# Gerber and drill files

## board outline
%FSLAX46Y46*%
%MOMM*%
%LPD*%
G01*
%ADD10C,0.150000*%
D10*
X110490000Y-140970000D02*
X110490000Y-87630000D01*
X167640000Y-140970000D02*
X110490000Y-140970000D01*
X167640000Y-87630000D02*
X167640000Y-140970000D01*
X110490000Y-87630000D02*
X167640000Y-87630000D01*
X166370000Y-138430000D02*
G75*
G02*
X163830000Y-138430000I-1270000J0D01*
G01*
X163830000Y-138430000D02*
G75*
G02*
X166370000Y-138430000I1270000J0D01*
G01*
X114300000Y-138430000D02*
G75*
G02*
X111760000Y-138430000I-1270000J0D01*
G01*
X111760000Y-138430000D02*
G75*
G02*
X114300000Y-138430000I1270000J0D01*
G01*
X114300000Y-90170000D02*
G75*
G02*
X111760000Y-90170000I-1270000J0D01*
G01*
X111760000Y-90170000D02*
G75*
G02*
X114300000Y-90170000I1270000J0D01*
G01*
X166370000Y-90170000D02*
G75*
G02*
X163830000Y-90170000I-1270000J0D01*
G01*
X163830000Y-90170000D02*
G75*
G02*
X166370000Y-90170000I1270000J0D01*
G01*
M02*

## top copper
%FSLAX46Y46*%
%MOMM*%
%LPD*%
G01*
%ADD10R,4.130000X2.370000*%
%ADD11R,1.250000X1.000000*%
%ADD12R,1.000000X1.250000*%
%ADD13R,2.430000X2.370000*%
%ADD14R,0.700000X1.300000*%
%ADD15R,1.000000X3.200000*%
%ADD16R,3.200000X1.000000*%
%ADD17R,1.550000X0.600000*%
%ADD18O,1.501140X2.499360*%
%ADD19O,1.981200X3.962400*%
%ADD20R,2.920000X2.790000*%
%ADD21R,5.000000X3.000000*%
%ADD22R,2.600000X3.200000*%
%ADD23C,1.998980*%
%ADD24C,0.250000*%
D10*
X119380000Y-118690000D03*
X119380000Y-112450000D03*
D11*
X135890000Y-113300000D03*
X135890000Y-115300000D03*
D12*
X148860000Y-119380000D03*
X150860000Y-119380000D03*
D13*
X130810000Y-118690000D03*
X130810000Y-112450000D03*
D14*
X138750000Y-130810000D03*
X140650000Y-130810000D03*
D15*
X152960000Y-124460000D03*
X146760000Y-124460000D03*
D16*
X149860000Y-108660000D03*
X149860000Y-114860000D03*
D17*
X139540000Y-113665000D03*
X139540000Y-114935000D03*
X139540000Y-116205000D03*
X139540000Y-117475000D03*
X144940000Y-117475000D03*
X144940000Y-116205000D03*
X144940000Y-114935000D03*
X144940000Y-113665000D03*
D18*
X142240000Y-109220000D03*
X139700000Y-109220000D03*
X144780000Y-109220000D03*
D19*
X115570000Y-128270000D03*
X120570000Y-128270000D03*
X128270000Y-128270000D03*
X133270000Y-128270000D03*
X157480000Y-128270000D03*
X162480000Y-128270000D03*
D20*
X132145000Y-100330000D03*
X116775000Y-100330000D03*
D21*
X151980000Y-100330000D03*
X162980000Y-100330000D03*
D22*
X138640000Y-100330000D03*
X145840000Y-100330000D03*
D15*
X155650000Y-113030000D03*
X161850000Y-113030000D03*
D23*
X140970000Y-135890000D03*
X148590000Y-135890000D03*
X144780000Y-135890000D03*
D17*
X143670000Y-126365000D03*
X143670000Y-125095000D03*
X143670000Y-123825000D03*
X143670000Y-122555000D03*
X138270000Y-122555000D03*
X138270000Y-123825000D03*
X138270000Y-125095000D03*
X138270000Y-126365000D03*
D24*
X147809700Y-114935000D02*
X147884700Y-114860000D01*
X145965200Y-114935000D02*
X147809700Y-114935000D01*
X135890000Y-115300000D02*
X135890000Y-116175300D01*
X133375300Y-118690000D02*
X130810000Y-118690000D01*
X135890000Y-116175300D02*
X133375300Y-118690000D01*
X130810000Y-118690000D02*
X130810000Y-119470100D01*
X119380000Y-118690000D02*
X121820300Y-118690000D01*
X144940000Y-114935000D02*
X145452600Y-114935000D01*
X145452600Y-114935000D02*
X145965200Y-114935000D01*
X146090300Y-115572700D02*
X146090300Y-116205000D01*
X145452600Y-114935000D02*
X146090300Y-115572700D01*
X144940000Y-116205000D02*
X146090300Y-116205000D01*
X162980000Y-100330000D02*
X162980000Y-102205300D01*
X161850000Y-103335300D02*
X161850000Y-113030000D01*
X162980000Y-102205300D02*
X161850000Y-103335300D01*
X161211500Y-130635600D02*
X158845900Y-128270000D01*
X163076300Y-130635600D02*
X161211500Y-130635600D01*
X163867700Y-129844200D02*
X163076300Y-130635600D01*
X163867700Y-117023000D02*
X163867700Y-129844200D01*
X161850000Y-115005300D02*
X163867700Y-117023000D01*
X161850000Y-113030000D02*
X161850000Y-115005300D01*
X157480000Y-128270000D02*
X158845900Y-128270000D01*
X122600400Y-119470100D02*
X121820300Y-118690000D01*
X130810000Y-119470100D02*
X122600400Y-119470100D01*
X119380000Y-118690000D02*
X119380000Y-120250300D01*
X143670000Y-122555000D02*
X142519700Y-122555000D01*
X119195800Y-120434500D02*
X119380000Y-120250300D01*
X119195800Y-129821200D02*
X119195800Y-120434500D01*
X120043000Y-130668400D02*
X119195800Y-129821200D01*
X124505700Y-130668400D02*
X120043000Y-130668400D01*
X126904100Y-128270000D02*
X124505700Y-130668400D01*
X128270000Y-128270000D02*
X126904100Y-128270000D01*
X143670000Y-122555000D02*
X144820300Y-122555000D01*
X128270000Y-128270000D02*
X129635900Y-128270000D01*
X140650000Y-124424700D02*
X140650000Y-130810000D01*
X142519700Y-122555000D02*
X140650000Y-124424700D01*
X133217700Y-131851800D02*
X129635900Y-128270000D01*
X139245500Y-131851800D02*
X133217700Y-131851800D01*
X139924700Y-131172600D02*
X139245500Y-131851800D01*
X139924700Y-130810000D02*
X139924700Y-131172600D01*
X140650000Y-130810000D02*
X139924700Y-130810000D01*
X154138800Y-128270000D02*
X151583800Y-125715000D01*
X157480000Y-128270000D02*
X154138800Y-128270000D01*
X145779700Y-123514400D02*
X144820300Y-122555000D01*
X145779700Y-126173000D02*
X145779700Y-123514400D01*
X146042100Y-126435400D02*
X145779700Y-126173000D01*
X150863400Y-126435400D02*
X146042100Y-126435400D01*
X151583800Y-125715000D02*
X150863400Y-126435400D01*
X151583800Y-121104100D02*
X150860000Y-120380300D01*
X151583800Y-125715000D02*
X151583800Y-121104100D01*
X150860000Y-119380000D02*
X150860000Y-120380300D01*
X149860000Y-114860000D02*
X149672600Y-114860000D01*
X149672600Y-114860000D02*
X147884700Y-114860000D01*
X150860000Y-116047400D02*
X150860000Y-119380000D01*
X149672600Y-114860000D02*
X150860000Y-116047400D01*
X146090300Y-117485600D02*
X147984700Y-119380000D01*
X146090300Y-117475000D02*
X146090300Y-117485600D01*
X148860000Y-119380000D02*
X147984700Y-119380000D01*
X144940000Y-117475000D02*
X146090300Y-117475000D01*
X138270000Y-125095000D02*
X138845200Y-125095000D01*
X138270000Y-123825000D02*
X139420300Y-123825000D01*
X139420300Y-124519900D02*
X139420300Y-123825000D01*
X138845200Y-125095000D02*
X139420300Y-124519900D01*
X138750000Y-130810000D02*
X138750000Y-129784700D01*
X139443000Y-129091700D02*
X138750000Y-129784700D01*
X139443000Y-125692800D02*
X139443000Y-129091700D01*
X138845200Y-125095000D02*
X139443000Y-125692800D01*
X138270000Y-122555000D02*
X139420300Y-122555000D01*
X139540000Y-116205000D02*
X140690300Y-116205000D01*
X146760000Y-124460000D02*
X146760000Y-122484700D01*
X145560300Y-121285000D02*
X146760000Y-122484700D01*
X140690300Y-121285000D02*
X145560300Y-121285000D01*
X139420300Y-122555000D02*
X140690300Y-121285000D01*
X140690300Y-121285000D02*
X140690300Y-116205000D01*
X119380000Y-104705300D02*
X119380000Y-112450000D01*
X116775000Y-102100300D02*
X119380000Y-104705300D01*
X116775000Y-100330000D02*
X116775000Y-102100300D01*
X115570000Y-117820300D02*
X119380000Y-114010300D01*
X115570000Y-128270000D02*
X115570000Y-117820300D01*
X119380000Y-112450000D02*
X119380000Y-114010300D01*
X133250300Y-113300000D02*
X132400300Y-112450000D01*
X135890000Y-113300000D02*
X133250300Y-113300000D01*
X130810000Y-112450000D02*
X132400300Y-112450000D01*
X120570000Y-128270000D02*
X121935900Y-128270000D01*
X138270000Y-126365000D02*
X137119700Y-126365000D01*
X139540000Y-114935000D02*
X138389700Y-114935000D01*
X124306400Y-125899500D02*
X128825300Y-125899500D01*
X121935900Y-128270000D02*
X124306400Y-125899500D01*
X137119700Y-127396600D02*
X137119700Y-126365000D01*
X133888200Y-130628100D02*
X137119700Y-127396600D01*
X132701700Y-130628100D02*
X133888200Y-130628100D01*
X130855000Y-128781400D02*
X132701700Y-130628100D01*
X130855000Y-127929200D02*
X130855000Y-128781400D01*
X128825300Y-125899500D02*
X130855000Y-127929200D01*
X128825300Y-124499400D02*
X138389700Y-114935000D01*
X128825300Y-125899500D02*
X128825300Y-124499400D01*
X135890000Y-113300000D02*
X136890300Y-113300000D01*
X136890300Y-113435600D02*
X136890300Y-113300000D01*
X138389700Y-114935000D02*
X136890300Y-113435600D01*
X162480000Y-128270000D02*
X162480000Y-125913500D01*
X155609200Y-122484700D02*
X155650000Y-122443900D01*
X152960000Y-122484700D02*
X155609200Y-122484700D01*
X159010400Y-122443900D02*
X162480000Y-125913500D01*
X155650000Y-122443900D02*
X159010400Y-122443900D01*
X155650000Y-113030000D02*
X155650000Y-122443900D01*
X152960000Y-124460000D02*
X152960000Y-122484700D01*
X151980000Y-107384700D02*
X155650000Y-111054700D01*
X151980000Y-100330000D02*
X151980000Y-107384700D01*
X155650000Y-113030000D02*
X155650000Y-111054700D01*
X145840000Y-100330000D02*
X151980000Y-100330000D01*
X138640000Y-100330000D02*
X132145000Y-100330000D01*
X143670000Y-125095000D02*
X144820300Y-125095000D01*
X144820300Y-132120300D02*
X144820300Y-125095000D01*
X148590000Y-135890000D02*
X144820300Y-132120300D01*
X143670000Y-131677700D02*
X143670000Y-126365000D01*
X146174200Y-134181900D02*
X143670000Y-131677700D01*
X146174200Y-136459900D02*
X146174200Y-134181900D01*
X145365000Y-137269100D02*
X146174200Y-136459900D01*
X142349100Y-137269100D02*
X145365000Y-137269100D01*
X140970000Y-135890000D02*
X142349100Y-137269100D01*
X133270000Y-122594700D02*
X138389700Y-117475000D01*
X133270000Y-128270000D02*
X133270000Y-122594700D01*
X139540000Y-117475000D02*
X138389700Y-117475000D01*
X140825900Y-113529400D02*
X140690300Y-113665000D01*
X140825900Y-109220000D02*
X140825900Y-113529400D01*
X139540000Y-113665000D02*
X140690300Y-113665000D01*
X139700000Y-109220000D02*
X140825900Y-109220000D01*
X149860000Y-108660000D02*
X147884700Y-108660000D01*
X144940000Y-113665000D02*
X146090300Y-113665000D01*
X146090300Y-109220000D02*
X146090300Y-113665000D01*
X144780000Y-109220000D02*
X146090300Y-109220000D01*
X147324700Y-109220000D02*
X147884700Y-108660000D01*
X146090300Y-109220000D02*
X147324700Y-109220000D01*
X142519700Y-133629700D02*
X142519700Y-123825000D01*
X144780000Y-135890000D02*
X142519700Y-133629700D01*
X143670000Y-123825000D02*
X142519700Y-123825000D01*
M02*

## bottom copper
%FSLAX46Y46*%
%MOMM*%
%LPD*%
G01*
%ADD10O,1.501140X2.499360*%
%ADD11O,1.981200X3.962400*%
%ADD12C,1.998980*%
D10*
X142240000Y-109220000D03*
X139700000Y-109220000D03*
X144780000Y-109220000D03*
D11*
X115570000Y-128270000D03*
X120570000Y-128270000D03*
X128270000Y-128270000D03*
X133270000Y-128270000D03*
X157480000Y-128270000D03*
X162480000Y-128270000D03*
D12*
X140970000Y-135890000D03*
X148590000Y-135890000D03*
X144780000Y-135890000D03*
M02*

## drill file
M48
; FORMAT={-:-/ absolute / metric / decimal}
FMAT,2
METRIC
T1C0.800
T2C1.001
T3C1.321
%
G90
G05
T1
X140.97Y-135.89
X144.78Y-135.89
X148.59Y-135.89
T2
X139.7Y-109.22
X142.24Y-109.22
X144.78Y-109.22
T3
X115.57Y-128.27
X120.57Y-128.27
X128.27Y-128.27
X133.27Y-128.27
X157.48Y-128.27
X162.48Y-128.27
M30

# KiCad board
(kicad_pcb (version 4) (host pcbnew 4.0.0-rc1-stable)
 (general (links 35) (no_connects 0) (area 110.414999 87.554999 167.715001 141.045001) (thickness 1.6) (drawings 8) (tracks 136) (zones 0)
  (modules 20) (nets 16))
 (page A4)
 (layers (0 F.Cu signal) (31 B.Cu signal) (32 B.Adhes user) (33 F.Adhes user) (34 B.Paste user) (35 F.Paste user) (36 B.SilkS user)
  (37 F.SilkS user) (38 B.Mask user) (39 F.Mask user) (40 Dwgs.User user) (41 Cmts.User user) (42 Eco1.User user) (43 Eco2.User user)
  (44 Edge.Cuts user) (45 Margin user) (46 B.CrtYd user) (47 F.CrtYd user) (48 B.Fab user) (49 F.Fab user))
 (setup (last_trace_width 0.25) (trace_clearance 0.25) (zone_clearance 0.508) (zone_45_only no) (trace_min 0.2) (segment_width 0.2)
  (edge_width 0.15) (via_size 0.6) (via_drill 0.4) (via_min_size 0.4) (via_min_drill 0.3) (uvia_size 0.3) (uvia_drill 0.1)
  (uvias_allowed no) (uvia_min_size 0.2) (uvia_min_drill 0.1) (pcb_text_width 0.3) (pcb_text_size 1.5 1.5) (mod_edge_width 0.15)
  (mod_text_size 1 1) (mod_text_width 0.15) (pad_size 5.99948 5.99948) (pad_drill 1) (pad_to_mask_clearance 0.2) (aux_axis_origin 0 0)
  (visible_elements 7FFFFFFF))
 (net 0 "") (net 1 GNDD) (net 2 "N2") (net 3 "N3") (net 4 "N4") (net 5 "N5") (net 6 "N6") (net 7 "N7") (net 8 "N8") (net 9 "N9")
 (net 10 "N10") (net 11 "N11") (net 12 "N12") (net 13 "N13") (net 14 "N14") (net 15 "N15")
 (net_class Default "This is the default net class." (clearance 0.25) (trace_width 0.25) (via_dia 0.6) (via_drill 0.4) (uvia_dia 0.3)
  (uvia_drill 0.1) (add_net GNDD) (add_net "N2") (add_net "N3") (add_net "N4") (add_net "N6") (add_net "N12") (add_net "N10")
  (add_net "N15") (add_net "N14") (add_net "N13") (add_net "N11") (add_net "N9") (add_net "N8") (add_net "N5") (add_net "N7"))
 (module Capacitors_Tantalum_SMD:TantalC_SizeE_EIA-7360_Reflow (layer F.Cu) (at 119.38 115.57 270)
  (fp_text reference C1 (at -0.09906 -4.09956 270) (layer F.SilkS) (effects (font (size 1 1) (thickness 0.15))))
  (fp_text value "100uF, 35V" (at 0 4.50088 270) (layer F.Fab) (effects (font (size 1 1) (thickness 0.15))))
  (pad 2 smd rect (at 3.12 0 270) (size 2.37 4.13) (layers F.Cu F.Paste F.Mask) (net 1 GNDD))
  (pad 1 smd rect (at -3.12 0 270) (size 2.37 4.13) (layers F.Cu F.Paste F.Mask) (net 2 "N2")))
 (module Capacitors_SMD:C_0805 (layer F.Cu) (at 135.89 114.3 270)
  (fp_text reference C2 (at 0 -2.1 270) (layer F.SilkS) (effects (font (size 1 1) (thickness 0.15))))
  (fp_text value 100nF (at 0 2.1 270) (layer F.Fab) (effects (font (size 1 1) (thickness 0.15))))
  (pad 1 smd rect (at -1 0 270) (size 1 1.25) (layers F.Cu F.Paste F.Mask) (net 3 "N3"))
  (pad 2 smd rect (at 1 0 270) (size 1 1.25) (layers F.Cu F.Paste F.Mask) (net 1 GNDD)))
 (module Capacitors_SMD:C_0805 (layer F.Cu) (at 149.86 119.38)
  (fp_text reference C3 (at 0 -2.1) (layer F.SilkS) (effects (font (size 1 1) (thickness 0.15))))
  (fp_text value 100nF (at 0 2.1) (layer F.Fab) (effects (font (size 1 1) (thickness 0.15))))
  (pad 1 smd rect (at -1 0) (size 1 1.25) (layers F.Cu F.Paste F.Mask) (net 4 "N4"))
  (pad 2 smd rect (at 1 0) (size 1 1.25) (layers F.Cu F.Paste F.Mask) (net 1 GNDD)))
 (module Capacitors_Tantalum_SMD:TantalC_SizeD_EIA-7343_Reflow (layer F.Cu) (at 130.81 115.57 270)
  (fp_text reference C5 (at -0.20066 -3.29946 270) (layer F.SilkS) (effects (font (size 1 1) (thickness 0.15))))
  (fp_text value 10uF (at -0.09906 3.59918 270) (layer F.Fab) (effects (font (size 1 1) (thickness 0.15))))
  (pad 2 smd rect (at 3.12 0 270) (size 2.37 2.43) (layers F.Cu F.Paste F.Mask) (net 1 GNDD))
  (pad 1 smd rect (at -3.12 0 270) (size 2.37 2.43) (layers F.Cu F.Paste F.Mask) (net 3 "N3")))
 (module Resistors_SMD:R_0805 (layer F.Cu) (at 139.7 130.81)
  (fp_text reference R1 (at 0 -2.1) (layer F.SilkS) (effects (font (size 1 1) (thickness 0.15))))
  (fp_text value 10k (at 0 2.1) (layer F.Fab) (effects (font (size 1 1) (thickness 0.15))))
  (pad 1 smd rect (at -0.95 0) (size 0.7 1.3) (layers F.Cu F.Paste F.Mask) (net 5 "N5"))
  (pad 2 smd rect (at 0.95 0) (size 0.7 1.3) (layers F.Cu F.Paste F.Mask) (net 1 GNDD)))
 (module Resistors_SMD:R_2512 (layer F.Cu) (at 149.86 124.46 180)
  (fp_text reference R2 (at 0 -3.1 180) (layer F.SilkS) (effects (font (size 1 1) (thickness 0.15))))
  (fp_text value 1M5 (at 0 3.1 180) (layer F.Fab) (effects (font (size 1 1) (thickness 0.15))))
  (pad 1 smd rect (at -3.1 0 180) (size 1 3.2) (layers F.Cu F.Paste F.Mask) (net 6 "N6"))
  (pad 2 smd rect (at 3.1 0 180) (size 1 3.2) (layers F.Cu F.Paste F.Mask) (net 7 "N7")))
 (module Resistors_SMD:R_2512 (layer F.Cu) (at 149.86 111.76 270)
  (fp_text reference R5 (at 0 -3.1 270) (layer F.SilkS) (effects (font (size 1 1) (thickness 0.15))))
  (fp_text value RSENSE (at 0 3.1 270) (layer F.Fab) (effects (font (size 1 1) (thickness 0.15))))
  (pad 1 smd rect (at -3.1 0 270) (size 1 3.2) (layers F.Cu F.Paste F.Mask) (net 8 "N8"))
  (pad 2 smd rect (at 3.1 0 270) (size 1 3.2) (layers F.Cu F.Paste F.Mask) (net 1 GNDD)))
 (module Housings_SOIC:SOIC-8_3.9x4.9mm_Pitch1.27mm (layer F.Cu) (at 142.24 115.57)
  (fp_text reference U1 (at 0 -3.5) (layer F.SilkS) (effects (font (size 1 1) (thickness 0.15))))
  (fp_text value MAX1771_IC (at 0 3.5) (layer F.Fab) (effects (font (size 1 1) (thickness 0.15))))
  (pad 1 smd rect (at -2.7 -1.905) (size 1.55 0.6) (layers F.Cu F.Paste F.Mask) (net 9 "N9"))
  (pad 2 smd rect (at -2.7 -0.635) (size 1.55 0.6) (layers F.Cu F.Paste F.Mask) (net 3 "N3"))
  (pad 3 smd rect (at -2.7 0.635) (size 1.55 0.6) (layers F.Cu F.Paste F.Mask) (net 7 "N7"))
  (pad 4 smd rect (at -2.7 1.905) (size 1.55 0.6) (layers F.Cu F.Paste F.Mask) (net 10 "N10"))
  (pad 5 smd rect (at 2.7 1.905) (size 1.55 0.6) (layers F.Cu F.Paste F.Mask) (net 4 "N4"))
  (pad 6 smd rect (at 2.7 0.635) (size 1.55 0.6) (layers F.Cu F.Paste F.Mask) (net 1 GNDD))
  (pad 7 smd rect (at 2.7 -0.635) (size 1.55 0.6) (layers F.Cu F.Paste F.Mask) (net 1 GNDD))
  (pad 8 smd rect (at 2.7 -1.905) (size 1.55 0.6) (layers F.Cu F.Paste F.Mask) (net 8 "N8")))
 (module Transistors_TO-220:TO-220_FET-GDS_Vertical (layer F.Cu) (at 142.24 109.22)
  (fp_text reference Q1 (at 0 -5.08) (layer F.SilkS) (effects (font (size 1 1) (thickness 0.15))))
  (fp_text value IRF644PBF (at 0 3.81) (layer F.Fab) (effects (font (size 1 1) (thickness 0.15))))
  (pad D thru_hole oval (at 0 0 90) (size 2.49936 1.50114) (drill 1.00076) (layers *.Cu *.Mask F.SilkS) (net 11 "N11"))
  (pad G thru_hole oval (at -2.54 0 90) (size 2.49936 1.50114) (drill 1.00076) (layers *.Cu *.Mask F.SilkS) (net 9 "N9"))
  (pad S thru_hole oval (at 2.54 0 90) (size 2.49936 1.50114) (drill 1.00076) (layers *.Cu *.Mask F.SilkS) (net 8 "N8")))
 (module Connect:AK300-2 (layer F.Cu) (at 115.57 128.27)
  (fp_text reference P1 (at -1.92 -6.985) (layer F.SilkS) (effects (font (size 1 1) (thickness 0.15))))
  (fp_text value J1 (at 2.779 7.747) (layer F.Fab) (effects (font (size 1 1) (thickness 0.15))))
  (pad 1 thru_hole oval (at 0 0) (size 1.9812 3.9624) (drill 1.3208) (layers *.Cu F.Paste F.SilkS F.Mask) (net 2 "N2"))
  (pad 2 thru_hole oval (at 5 0) (size 1.9812 3.9624) (drill 1.3208) (layers *.Cu F.Paste F.SilkS F.Mask) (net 3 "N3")))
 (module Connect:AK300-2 (layer F.Cu) (at 128.27 128.27)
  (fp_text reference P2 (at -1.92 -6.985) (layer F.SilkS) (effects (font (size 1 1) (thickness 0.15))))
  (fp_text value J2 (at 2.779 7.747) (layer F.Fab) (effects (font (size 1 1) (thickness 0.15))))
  (pad 1 thru_hole oval (at 0 0) (size 1.9812 3.9624) (drill 1.3208) (layers *.Cu F.Paste F.SilkS F.Mask) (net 1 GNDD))
  (pad 2 thru_hole oval (at 5 0) (size 1.9812 3.9624) (drill 1.3208) (layers *.Cu F.Paste F.SilkS F.Mask) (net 10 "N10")))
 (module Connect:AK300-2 (layer F.Cu) (at 157.48 128.27)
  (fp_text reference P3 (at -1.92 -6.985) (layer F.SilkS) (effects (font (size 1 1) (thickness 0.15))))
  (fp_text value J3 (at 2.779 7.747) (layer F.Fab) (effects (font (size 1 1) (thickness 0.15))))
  (pad 1 thru_hole oval (at 0 0) (size 1.9812 3.9624) (drill 1.3208) (layers *.Cu F.Paste F.SilkS F.Mask) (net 1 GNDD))
  (pad 2 thru_hole oval (at 5 0) (size 1.9812 3.9624) (drill 1.3208) (layers *.Cu F.Paste F.SilkS F.Mask) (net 6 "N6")))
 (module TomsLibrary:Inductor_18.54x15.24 (layer F.Cu) (at 124.46 100.33 180)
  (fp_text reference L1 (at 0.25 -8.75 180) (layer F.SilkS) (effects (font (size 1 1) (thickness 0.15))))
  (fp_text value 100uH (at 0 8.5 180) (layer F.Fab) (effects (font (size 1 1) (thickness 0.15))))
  (pad 1 smd rect (at -7.685 0 180) (size 2.92 2.79) (layers F.Cu F.Paste F.Mask) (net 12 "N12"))
  (pad 2 smd rect (at 7.685 0 180) (size 2.92 2.79) (layers F.Cu F.Paste F.Mask) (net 2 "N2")))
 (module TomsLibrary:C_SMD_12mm (layer F.Cu) (at 157.48 100.33 180)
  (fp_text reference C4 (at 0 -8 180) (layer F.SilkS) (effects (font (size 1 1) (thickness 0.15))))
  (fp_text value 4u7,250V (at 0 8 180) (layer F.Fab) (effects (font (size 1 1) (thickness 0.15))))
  (pad 1 smd rect (at 5.5 0 180) (size 5 3) (layers F.Cu F.Paste F.Mask) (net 6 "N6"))
  (pad 2 smd rect (at -5.5 0 180) (size 5 3) (layers F.Cu F.Paste F.Mask) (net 1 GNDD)))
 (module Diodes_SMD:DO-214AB (layer F.Cu) (at 142.24 100.33 180)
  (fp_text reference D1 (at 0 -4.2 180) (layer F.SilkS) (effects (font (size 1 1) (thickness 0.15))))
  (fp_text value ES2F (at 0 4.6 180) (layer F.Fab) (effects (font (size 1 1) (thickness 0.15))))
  (pad 2 smd rect (at 3.6 0 180) (size 2.6 3.2) (layers F.Cu F.Paste F.Mask) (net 12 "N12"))
  (pad 1 smd rect (at -3.6 0 180) (size 2.6 3.2) (layers F.Cu F.Paste F.Mask) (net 6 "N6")))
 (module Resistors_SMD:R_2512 (layer F.Cu) (at 158.75 113.03)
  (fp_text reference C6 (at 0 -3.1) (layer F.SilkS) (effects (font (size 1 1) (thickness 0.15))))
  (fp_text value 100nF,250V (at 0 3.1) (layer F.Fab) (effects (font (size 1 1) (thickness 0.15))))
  (pad 1 smd rect (at -3.1 0) (size 1 3.2) (layers F.Cu F.Paste F.Mask) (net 6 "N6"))
  (pad 2 smd rect (at 3.1 0) (size 1 3.2) (layers F.Cu F.Paste F.Mask) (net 1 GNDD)))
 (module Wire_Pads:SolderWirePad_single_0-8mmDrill (layer F.Cu) (at 140.97 135.89)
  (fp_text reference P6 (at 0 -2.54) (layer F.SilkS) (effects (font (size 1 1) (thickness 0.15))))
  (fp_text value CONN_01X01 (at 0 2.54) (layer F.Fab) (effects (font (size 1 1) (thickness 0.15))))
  (pad 1 thru_hole circle (at 0 0) (size 1.99898 1.99898) (drill 0.8001) (layers *.Cu *.Mask F.SilkS) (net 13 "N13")))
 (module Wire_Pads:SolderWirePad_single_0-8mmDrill (layer F.Cu) (at 148.59 135.89)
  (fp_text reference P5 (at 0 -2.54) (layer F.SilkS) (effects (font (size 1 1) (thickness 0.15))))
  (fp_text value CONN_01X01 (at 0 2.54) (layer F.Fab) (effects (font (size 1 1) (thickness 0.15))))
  (pad 1 thru_hole circle (at 0 0) (size 1.99898 1.99898) (drill 0.8001) (layers *.Cu *.Mask F.SilkS) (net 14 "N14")))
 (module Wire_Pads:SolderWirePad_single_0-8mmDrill (layer F.Cu) (at 144.78 135.89)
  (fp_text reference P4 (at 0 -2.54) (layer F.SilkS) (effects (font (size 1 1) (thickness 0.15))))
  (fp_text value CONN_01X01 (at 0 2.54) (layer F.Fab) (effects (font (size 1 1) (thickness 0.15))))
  (pad 1 thru_hole circle (at 0 0) (size 1.99898 1.99898) (drill 0.8001) (layers *.Cu *.Mask F.SilkS) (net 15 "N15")))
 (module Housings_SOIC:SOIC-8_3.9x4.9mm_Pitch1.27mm (layer F.Cu) (at 140.97 124.46 180)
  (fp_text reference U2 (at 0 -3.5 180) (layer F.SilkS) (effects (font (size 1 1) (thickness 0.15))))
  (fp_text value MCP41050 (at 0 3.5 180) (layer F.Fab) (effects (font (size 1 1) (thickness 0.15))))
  (pad 1 smd rect (at -2.7 -1.905 180) (size 1.55 0.6) (layers F.Cu F.Paste F.Mask) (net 13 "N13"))
  (pad 2 smd rect (at -2.7 -0.635 180) (size 1.55 0.6) (layers F.Cu F.Paste F.Mask) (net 14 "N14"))
  (pad 3 smd rect (at -2.7 0.635 180) (size 1.55 0.6) (layers F.Cu F.Paste F.Mask) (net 15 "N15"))
  (pad 4 smd rect (at -2.7 1.905 180) (size 1.55 0.6) (layers F.Cu F.Paste F.Mask) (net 1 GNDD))
  (pad 5 smd rect (at 2.7 1.905 180) (size 1.55 0.6) (layers F.Cu F.Paste F.Mask) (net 7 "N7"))
  (pad 6 smd rect (at 2.7 0.635 180) (size 1.55 0.6) (layers F.Cu F.Paste F.Mask) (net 5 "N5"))
  (pad 7 smd rect (at 2.7 -0.635 180) (size 1.55 0.6) (layers F.Cu F.Paste F.Mask) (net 5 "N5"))
  (pad 8 smd rect (at 2.7 -1.905 180) (size 1.55 0.6) (layers F.Cu F.Paste F.Mask) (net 3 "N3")))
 (gr_line (start 110.49 140.97) (end 110.49 87.63) (angle 90) (layer Edge.Cuts) (width 0.15))
 (gr_line (start 167.64 140.97) (end 110.49 140.97) (angle 90) (layer Edge.Cuts) (width 0.15))
 (gr_line (start 167.64 87.63) (end 167.64 140.97) (angle 90) (layer Edge.Cuts) (width 0.15))
 (gr_line (start 110.49 87.63) (end 167.64 87.63) (angle 90) (layer Edge.Cuts) (width 0.15))
 (gr_circle (center 165.1 138.43) (end 163.83 138.43) (layer Edge.Cuts) (width 0.15))
 (gr_circle (center 113.03 138.43) (end 114.3 138.43) (layer Edge.Cuts) (width 0.15))
 (gr_circle (center 113.03 90.17) (end 114.3 90.17) (layer Edge.Cuts) (width 0.15))
 (gr_circle (center 165.1 90.17) (end 163.83 90.17) (layer Edge.Cuts) (width 0.15))
 (segment (start 147.8097 114.935) (end 147.8847 114.86) (width 0.25) (layer F.Cu) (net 1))
 (segment (start 145.9652 114.935) (end 147.8097 114.935) (width 0.25) (layer F.Cu) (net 1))
 (segment (start 135.89 115.3) (end 135.89 116.1753) (width 0.25) (layer F.Cu) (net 1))
 (segment (start 133.3753 118.69) (end 130.81 118.69) (width 0.25) (layer F.Cu) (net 1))
 (segment (start 135.89 116.1753) (end 133.3753 118.69) (width 0.25) (layer F.Cu) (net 1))
 (segment (start 130.81 118.69) (end 130.81 119.4701) (width 0.25) (layer F.Cu) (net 1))
 (segment (start 119.38 118.69) (end 121.8203 118.69) (width 0.25) (layer F.Cu) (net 1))
 (segment (start 144.94 114.935) (end 145.4526 114.935) (width 0.25) (layer F.Cu) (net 1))
 (segment (start 145.4526 114.935) (end 145.9652 114.935) (width 0.25) (layer F.Cu) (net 1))
 (segment (start 146.0903 115.5727) (end 146.0903 116.205) (width 0.25) (layer F.Cu) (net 1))
 (segment (start 145.4526 114.935) (end 146.0903 115.5727) (width 0.25) (layer F.Cu) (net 1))
 (segment (start 144.94 116.205) (end 146.0903 116.205) (width 0.25) (layer F.Cu) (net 1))
 (segment (start 162.98 100.33) (end 162.98 102.2053) (width 0.25) (layer F.Cu) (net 1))
 (segment (start 161.85 103.3353) (end 161.85 113.03) (width 0.25) (layer F.Cu) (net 1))
 (segment (start 162.98 102.2053) (end 161.85 103.3353) (width 0.25) (layer F.Cu) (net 1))
 (segment (start 161.2115 130.6356) (end 158.8459 128.27) (width 0.25) (layer F.Cu) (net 1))
 (segment (start 163.0763 130.6356) (end 161.2115 130.6356) (width 0.25) (layer F.Cu) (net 1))
 (segment (start 163.8677 129.8442) (end 163.0763 130.6356) (width 0.25) (layer F.Cu) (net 1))
 (segment (start 163.8677 117.023) (end 163.8677 129.8442) (width 0.25) (layer F.Cu) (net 1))
 (segment (start 161.85 115.0053) (end 163.8677 117.023) (width 0.25) (layer F.Cu) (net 1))
 (segment (start 161.85 113.03) (end 161.85 115.0053) (width 0.25) (layer F.Cu) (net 1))
 (segment (start 157.48 128.27) (end 158.8459 128.27) (width 0.25) (layer F.Cu) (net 1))
 (segment (start 122.6004 119.4701) (end 121.8203 118.69) (width 0.25) (layer F.Cu) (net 1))
 (segment (start 130.81 119.4701) (end 122.6004 119.4701) (width 0.25) (layer F.Cu) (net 1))
 (segment (start 119.38 118.69) (end 119.38 120.2503) (width 0.25) (layer F.Cu) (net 1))
 (segment (start 143.67 122.555) (end 142.5197 122.555) (width 0.25) (layer F.Cu) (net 1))
 (segment (start 119.1958 120.4345) (end 119.38 120.2503) (width 0.25) (layer F.Cu) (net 1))
 (segment (start 119.1958 129.8212) (end 119.1958 120.4345) (width 0.25) (layer F.Cu) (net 1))
 (segment (start 120.043 130.6684) (end 119.1958 129.8212) (width 0.25) (layer F.Cu) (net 1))
 (segment (start 124.5057 130.6684) (end 120.043 130.6684) (width 0.25) (layer F.Cu) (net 1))
 (segment (start 126.9041 128.27) (end 124.5057 130.6684) (width 0.25) (layer F.Cu) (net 1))
 (segment (start 128.27 128.27) (end 126.9041 128.27) (width 0.25) (layer F.Cu) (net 1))
 (segment (start 143.67 122.555) (end 144.8203 122.555) (width 0.25) (layer F.Cu) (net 1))
 (segment (start 128.27 128.27) (end 129.6359 128.27) (width 0.25) (layer F.Cu) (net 1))
 (segment (start 140.65 124.4247) (end 140.65 130.81) (width 0.25) (layer F.Cu) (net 1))
 (segment (start 142.5197 122.555) (end 140.65 124.4247) (width 0.25) (layer F.Cu) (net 1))
 (segment (start 133.2177 131.8518) (end 129.6359 128.27) (width 0.25) (layer F.Cu) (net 1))
 (segment (start 139.2455 131.8518) (end 133.2177 131.8518) (width 0.25) (layer F.Cu) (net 1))
 (segment (start 139.9247 131.1726) (end 139.2455 131.8518) (width 0.25) (layer F.Cu) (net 1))
 (segment (start 139.9247 130.81) (end 139.9247 131.1726) (width 0.25) (layer F.Cu) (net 1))
 (segment (start 140.65 130.81) (end 139.9247 130.81) (width 0.25) (layer F.Cu) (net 1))
 (segment (start 154.1388 128.27) (end 151.5838 125.715) (width 0.25) (layer F.Cu) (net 1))
 (segment (start 157.48 128.27) (end 154.1388 128.27) (width 0.25) (layer F.Cu) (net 1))
 (segment (start 145.7797 123.5144) (end 144.8203 122.555) (width 0.25) (layer F.Cu) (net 1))
 (segment (start 145.7797 126.173) (end 145.7797 123.5144) (width 0.25) (layer F.Cu) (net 1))
 (segment (start 146.0421 126.4354) (end 145.7797 126.173) (width 0.25) (layer F.Cu) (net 1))
 (segment (start 150.8634 126.4354) (end 146.0421 126.4354) (width 0.25) (layer F.Cu) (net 1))
 (segment (start 151.5838 125.715) (end 150.8634 126.4354) (width 0.25) (layer F.Cu) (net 1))
 (segment (start 151.5838 121.1041) (end 150.86 120.3803) (width 0.25) (layer F.Cu) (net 1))
 (segment (start 151.5838 125.715) (end 151.5838 121.1041) (width 0.25) (layer F.Cu) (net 1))
 (segment (start 150.86 119.38) (end 150.86 120.3803) (width 0.25) (layer F.Cu) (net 1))
 (segment (start 149.86 114.86) (end 149.6726 114.86) (width 0.25) (layer F.Cu) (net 1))
 (segment (start 149.6726 114.86) (end 147.8847 114.86) (width 0.25) (layer F.Cu) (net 1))
 (segment (start 150.86 116.0474) (end 150.86 119.38) (width 0.25) (layer F.Cu) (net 1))
 (segment (start 149.6726 114.86) (end 150.86 116.0474) (width 0.25) (layer F.Cu) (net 1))
 (segment (start 146.0903 117.4856) (end 147.9847 119.38) (width 0.25) (layer F.Cu) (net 4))
 (segment (start 146.0903 117.475) (end 146.0903 117.4856) (width 0.25) (layer F.Cu) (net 4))
 (segment (start 148.86 119.38) (end 147.9847 119.38) (width 0.25) (layer F.Cu) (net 4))
 (segment (start 144.94 117.475) (end 146.0903 117.475) (width 0.25) (layer F.Cu) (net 4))
 (segment (start 138.27 125.095) (end 138.8452 125.095) (width 0.25) (layer F.Cu) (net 5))
 (segment (start 138.27 123.825) (end 139.4203 123.825) (width 0.25) (layer F.Cu) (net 5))
 (segment (start 139.4203 124.5199) (end 139.4203 123.825) (width 0.25) (layer F.Cu) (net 5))
 (segment (start 138.8452 125.095) (end 139.4203 124.5199) (width 0.25) (layer F.Cu) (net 5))
 (segment (start 138.75 130.81) (end 138.75 129.7847) (width 0.25) (layer F.Cu) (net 5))
 (segment (start 139.443 129.0917) (end 138.75 129.7847) (width 0.25) (layer F.Cu) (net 5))
 (segment (start 139.443 125.6928) (end 139.443 129.0917) (width 0.25) (layer F.Cu) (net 5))
 (segment (start 138.8452 125.095) (end 139.443 125.6928) (width 0.25) (layer F.Cu) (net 5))
 (segment (start 138.27 122.555) (end 139.4203 122.555) (width 0.25) (layer F.Cu) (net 7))
 (segment (start 139.54 116.205) (end 140.6903 116.205) (width 0.25) (layer F.Cu) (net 7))
 (segment (start 146.76 124.46) (end 146.76 122.4847) (width 0.25) (layer F.Cu) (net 7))
 (segment (start 145.5603 121.285) (end 146.76 122.4847) (width 0.25) (layer F.Cu) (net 7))
 (segment (start 140.6903 121.285) (end 145.5603 121.285) (width 0.25) (layer F.Cu) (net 7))
 (segment (start 139.4203 122.555) (end 140.6903 121.285) (width 0.25) (layer F.Cu) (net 7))
 (segment (start 140.6903 121.285) (end 140.6903 116.205) (width 0.25) (layer F.Cu) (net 7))
 (segment (start 119.38 104.7053) (end 119.38 112.45) (width 0.25) (layer F.Cu) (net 2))
 (segment (start 116.775 102.1003) (end 119.38 104.7053) (width 0.25) (layer F.Cu) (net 2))
 (segment (start 116.775 100.33) (end 116.775 102.1003) (width 0.25) (layer F.Cu) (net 2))
 (segment (start 115.57 117.8203) (end 119.38 114.0103) (width 0.25) (layer F.Cu) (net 2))
 (segment (start 115.57 128.27) (end 115.57 117.8203) (width 0.25) (layer F.Cu) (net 2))
 (segment (start 119.38 112.45) (end 119.38 114.0103) (width 0.25) (layer F.Cu) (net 2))
 (segment (start 133.2503 113.3) (end 132.4003 112.45) (width 0.25) (layer F.Cu) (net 3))
 (segment (start 135.89 113.3) (end 133.2503 113.3) (width 0.25) (layer F.Cu) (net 3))
 (segment (start 130.81 112.45) (end 132.4003 112.45) (width 0.25) (layer F.Cu) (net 3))
 (segment (start 120.57 128.27) (end 121.9359 128.27) (width 0.25) (layer F.Cu) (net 3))
 (segment (start 138.27 126.365) (end 137.1197 126.365) (width 0.25) (layer F.Cu) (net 3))
 (segment (start 139.54 114.935) (end 138.3897 114.935) (width 0.25) (layer F.Cu) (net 3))
 (segment (start 124.3064 125.8995) (end 128.8253 125.8995) (width 0.25) (layer F.Cu) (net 3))
 (segment (start 121.9359 128.27) (end 124.3064 125.8995) (width 0.25) (layer F.Cu) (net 3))
 (segment (start 137.1197 127.3966) (end 137.1197 126.365) (width 0.25) (layer F.Cu) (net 3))
 (segment (start 133.8882 130.6281) (end 137.1197 127.3966) (width 0.25) (layer F.Cu) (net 3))
 (segment (start 132.7017 130.6281) (end 133.8882 130.6281) (width 0.25) (layer F.Cu) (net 3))
 (segment (start 130.855 128.7814) (end 132.7017 130.6281) (width 0.25) (layer F.Cu) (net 3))
 (segment (start 130.855 127.9292) (end 130.855 128.7814) (width 0.25) (layer F.Cu) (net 3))
 (segment (start 128.8253 125.8995) (end 130.855 127.9292) (width 0.25) (layer F.Cu) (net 3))
 (segment (start 128.8253 124.4994) (end 138.3897 114.935) (width 0.25) (layer F.Cu) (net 3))
 (segment (start 128.8253 125.8995) (end 128.8253 124.4994) (width 0.25) (layer F.Cu) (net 3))
 (segment (start 135.89 113.3) (end 136.8903 113.3) (width 0.25) (layer F.Cu) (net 3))
 (segment (start 136.8903 113.4356) (end 136.8903 113.3) (width 0.25) (layer F.Cu) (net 3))
 (segment (start 138.3897 114.935) (end 136.8903 113.4356) (width 0.25) (layer F.Cu) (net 3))
 (segment (start 162.48 128.27) (end 162.48 125.9135) (width 0.25) (layer F.Cu) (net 6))
 (segment (start 155.6092 122.4847) (end 155.65 122.4439) (width 0.25) (layer F.Cu) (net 6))
 (segment (start 152.96 122.4847) (end 155.6092 122.4847) (width 0.25) (layer F.Cu) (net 6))
 (segment (start 159.0104 122.4439) (end 162.48 125.9135) (width 0.25) (layer F.Cu) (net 6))
 (segment (start 155.65 122.4439) (end 159.0104 122.4439) (width 0.25) (layer F.Cu) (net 6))
 (segment (start 155.65 113.03) (end 155.65 122.4439) (width 0.25) (layer F.Cu) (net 6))
 (segment (start 152.96 124.46) (end 152.96 122.4847) (width 0.25) (layer F.Cu) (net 6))
 (segment (start 151.98 107.3847) (end 155.65 111.0547) (width 0.25) (layer F.Cu) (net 6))
 (segment (start 151.98 100.33) (end 151.98 107.3847) (width 0.25) (layer F.Cu) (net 6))
 (segment (start 155.65 113.03) (end 155.65 111.0547) (width 0.25) (layer F.Cu) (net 6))
 (segment (start 145.84 100.33) (end 151.98 100.33) (width 0.25) (layer F.Cu) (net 6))
 (segment (start 138.64 100.33) (end 132.145 100.33) (width 0.25) (layer F.Cu) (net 12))
 (segment (start 143.67 125.095) (end 144.8203 125.095) (width 0.25) (layer F.Cu) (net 14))
 (segment (start 144.8203 132.1203) (end 144.8203 125.095) (width 0.25) (layer F.Cu) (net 14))
 (segment (start 148.59 135.89) (end 144.8203 132.1203) (width 0.25) (layer F.Cu) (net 14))
 (segment (start 143.67 131.6777) (end 143.67 126.365) (width 0.25) (layer F.Cu) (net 13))
 (segment (start 146.1742 134.1819) (end 143.67 131.6777) (width 0.25) (layer F.Cu) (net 13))
 (segment (start 146.1742 136.4599) (end 146.1742 134.1819) (width 0.25) (layer F.Cu) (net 13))
 (segment (start 145.365 137.2691) (end 146.1742 136.4599) (width 0.25) (layer F.Cu) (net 13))
 (segment (start 142.3491 137.2691) (end 145.365 137.2691) (width 0.25) (layer F.Cu) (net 13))
 (segment (start 140.97 135.89) (end 142.3491 137.2691) (width 0.25) (layer F.Cu) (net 13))
 (segment (start 133.27 122.5947) (end 138.3897 117.475) (width 0.25) (layer F.Cu) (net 10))
 (segment (start 133.27 128.27) (end 133.27 122.5947) (width 0.25) (layer F.Cu) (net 10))
 (segment (start 139.54 117.475) (end 138.3897 117.475) (width 0.25) (layer F.Cu) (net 10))
 (segment (start 140.8259 113.5294) (end 140.6903 113.665) (width 0.25) (layer F.Cu) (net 9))
 (segment (start 140.8259 109.22) (end 140.8259 113.5294) (width 0.25) (layer F.Cu) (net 9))
 (segment (start 139.54 113.665) (end 140.6903 113.665) (width 0.25) (layer F.Cu) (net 9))
 (segment (start 139.7 109.22) (end 140.8259 109.22) (width 0.25) (layer F.Cu) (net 9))
 (segment (start 149.86 108.66) (end 147.8847 108.66) (width 0.25) (layer F.Cu) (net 8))
 (segment (start 144.94 113.665) (end 146.0903 113.665) (width 0.25) (layer F.Cu) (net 8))
 (segment (start 146.0903 109.22) (end 146.0903 113.665) (width 0.25) (layer F.Cu) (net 8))
 (segment (start 144.78 109.22) (end 146.0903 109.22) (width 0.25) (layer F.Cu) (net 8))
 (segment (start 147.3247 109.22) (end 147.8847 108.66) (width 0.25) (layer F.Cu) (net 8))
 (segment (start 146.0903 109.22) (end 147.3247 109.22) (width 0.25) (layer F.Cu) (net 8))
 (segment (start 142.5197 133.6297) (end 142.5197 123.825) (width 0.25) (layer F.Cu) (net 15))
 (segment (start 144.78 135.89) (end 142.5197 133.6297) (width 0.25) (layer F.Cu) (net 15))
 (segment (start 143.67 123.825) (end 142.5197 123.825) (width 0.25) (layer F.Cu) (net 15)))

